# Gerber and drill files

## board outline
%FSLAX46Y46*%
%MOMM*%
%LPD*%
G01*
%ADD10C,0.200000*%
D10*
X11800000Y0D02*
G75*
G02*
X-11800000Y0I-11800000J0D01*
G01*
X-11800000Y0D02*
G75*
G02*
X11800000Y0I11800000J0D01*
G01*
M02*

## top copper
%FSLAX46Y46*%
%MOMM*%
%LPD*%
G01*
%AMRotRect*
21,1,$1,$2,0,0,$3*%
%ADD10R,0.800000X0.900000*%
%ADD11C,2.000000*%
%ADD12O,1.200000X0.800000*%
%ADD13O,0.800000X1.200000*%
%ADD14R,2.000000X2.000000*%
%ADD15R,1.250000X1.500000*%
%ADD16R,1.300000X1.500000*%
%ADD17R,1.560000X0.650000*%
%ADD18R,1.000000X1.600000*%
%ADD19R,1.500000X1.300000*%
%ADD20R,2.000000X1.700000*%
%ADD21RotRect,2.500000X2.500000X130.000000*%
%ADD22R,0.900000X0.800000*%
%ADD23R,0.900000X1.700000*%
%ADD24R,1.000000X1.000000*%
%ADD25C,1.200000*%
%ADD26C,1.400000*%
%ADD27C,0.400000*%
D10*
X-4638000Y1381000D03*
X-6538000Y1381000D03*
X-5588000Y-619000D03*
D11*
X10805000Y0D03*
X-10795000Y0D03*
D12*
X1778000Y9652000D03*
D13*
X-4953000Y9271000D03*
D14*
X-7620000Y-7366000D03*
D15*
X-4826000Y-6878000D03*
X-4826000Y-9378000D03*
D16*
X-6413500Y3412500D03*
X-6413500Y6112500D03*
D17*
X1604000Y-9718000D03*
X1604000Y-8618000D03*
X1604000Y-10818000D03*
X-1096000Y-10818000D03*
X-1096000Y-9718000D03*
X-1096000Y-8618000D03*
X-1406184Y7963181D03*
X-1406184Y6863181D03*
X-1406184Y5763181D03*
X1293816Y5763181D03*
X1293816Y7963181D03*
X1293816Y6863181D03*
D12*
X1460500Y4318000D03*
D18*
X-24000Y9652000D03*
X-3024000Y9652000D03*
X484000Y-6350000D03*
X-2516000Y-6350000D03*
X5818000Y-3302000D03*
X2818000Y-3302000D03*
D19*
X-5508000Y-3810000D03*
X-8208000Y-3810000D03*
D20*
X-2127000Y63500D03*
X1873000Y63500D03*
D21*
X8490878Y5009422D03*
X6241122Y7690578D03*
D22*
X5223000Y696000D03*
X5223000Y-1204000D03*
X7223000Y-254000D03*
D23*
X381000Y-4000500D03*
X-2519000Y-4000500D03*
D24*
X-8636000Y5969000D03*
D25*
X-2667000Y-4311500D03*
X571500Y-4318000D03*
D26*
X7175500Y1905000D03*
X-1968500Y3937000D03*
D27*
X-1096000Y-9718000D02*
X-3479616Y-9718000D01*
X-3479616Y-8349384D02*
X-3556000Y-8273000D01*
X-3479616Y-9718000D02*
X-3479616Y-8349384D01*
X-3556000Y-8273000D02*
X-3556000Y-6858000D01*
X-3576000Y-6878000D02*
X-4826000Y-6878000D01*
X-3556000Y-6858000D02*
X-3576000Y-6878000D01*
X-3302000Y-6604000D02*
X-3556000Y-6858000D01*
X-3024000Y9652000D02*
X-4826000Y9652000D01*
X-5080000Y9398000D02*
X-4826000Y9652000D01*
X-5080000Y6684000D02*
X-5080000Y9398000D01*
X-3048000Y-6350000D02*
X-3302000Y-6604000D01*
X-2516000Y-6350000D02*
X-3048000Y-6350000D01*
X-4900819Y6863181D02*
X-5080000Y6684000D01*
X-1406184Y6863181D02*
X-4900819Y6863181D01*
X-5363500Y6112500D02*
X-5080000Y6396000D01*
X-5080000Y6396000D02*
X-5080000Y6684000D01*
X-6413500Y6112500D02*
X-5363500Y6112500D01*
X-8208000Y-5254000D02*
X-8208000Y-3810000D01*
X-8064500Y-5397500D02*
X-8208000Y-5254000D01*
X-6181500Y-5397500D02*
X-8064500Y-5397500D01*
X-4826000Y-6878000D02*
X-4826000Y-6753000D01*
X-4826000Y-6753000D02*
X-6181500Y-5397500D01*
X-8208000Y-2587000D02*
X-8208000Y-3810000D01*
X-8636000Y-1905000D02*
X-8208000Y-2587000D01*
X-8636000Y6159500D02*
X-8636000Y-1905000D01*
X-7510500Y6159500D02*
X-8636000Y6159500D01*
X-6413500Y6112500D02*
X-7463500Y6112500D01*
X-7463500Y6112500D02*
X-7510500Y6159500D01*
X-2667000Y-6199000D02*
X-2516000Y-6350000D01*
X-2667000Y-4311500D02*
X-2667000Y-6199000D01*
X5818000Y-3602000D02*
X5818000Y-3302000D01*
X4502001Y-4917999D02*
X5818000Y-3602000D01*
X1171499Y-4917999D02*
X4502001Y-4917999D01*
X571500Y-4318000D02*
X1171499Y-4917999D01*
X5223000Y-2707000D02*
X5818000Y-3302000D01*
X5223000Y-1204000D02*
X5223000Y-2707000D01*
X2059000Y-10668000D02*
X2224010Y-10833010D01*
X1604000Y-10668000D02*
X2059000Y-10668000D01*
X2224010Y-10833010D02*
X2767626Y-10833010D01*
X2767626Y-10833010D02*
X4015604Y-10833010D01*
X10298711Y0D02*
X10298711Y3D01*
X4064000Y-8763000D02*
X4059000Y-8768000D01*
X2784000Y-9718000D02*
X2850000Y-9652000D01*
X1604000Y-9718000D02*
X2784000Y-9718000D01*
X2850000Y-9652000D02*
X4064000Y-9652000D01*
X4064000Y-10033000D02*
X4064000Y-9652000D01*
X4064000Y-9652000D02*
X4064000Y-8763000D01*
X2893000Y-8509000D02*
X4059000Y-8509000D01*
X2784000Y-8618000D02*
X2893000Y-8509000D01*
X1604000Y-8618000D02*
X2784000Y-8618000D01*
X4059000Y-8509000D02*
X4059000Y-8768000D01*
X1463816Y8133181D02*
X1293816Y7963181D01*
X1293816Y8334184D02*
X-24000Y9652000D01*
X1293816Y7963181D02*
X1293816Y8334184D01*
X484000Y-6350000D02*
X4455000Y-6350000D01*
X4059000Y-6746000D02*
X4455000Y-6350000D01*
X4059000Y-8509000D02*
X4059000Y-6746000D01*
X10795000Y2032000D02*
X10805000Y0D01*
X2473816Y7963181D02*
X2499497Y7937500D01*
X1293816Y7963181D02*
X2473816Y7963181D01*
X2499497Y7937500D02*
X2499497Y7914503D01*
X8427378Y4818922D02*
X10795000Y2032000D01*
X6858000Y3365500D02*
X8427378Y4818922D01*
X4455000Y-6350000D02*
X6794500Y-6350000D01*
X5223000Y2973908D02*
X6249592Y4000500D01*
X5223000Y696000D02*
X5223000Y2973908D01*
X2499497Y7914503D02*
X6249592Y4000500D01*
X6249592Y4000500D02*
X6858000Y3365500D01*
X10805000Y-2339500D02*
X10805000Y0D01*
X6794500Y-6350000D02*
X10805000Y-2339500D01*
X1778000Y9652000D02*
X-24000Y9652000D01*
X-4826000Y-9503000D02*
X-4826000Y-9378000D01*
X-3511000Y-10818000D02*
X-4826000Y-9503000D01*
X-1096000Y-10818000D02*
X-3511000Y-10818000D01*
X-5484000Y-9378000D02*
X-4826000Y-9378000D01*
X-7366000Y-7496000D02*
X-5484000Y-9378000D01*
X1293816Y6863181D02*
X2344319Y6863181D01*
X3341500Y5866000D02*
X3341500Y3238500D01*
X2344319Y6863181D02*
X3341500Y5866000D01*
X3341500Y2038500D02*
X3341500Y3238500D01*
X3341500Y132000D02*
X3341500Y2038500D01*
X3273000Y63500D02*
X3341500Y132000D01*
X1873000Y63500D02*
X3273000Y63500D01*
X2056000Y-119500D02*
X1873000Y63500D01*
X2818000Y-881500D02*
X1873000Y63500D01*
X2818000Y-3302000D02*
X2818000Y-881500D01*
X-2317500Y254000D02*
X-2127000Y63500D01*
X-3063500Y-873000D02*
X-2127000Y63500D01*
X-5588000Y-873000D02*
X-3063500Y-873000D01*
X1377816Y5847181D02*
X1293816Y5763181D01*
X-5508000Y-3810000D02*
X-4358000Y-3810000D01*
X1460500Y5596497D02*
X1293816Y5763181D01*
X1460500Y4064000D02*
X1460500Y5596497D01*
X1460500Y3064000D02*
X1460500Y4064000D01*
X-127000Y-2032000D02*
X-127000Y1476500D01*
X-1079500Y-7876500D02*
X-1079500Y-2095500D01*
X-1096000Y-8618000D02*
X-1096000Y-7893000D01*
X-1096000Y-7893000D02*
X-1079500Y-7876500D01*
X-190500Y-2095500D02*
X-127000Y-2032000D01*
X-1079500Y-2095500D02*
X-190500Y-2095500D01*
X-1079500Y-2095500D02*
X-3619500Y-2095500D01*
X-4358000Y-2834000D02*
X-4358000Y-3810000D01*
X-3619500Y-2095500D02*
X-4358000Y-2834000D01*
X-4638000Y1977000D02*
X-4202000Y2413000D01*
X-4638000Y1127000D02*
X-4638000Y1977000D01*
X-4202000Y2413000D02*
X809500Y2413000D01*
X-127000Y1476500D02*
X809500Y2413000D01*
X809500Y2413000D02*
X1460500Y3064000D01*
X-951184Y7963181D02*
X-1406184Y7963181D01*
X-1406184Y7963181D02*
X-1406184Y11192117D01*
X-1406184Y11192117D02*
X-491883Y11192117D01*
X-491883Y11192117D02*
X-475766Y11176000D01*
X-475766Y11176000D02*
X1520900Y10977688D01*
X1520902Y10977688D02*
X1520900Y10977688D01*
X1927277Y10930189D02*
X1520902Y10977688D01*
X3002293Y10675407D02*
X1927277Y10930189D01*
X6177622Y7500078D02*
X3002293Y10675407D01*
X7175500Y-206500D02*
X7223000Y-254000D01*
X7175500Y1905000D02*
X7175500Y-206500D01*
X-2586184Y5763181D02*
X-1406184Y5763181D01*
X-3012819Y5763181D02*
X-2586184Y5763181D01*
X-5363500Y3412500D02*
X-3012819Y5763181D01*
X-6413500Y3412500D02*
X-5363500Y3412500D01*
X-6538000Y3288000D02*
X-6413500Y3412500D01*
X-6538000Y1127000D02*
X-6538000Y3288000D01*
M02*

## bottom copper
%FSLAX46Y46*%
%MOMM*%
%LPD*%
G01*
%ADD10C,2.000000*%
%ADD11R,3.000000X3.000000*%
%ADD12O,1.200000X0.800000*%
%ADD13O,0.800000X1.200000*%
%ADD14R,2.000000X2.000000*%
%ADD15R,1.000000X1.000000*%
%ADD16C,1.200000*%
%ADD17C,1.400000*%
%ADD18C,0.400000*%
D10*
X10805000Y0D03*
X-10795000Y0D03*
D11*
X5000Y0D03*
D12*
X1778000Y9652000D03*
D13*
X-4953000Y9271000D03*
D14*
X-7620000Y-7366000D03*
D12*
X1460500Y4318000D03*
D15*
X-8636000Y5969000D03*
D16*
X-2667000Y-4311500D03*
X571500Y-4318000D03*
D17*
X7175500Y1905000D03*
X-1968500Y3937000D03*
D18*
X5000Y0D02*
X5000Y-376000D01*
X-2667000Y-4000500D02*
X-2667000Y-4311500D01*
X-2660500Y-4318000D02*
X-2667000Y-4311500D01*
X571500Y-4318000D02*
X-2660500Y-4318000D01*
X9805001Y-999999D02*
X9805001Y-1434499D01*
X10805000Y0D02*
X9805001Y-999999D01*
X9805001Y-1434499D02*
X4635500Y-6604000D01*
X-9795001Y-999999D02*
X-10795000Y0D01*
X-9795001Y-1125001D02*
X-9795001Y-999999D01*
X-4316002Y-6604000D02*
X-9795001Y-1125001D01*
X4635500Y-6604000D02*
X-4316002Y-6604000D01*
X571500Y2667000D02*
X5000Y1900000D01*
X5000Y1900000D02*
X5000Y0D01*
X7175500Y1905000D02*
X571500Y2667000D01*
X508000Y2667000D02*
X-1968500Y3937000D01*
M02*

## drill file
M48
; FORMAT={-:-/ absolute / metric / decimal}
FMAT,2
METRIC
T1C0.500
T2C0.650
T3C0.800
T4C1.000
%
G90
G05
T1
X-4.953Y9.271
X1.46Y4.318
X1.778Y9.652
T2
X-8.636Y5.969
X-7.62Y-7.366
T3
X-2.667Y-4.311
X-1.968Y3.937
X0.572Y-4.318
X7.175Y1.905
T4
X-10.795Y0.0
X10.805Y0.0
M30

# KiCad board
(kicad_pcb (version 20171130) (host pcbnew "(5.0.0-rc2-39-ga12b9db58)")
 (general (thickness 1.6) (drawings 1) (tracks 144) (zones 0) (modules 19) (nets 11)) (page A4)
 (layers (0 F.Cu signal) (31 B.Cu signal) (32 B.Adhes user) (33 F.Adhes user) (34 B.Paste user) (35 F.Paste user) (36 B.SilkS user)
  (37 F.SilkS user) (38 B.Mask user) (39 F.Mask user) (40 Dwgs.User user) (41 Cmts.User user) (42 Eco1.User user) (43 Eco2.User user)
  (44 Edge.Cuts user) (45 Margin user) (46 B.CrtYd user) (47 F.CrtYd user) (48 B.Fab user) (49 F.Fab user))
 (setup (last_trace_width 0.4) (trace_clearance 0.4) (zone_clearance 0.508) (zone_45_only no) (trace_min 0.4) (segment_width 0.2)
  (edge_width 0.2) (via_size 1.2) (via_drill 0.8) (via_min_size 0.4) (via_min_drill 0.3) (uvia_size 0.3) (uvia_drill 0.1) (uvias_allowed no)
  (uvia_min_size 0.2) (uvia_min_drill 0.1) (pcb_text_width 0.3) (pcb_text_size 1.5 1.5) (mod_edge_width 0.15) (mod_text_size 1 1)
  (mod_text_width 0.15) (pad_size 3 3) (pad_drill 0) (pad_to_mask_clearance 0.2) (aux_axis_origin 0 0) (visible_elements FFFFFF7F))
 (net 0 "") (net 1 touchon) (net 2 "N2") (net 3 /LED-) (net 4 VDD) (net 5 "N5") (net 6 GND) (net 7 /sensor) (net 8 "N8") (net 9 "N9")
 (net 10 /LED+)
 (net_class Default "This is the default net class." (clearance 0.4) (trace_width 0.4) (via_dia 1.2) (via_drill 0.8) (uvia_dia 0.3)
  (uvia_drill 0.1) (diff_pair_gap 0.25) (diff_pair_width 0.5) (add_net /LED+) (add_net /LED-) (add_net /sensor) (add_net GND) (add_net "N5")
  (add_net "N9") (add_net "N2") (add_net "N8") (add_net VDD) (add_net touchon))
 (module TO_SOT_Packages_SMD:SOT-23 (layer F.Cu) (at -5.588 -0.381 270)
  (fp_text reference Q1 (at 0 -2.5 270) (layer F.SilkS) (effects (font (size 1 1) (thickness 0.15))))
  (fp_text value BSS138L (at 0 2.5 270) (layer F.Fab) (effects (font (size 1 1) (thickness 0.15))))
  (pad 1 smd rect (at -1 -0.95 270) (size 0.9 0.8) (layers F.Cu F.Paste F.Mask) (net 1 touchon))
  (pad 2 smd rect (at -1 0.95 270) (size 0.9 0.8) (layers F.Cu F.Paste F.Mask) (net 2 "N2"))
  (pad 3 smd rect (at 1 0 270) (size 0.9 0.8) (layers F.Cu F.Paste F.Mask) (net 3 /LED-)))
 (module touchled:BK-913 (layer B.Cu) (at 0.005 0)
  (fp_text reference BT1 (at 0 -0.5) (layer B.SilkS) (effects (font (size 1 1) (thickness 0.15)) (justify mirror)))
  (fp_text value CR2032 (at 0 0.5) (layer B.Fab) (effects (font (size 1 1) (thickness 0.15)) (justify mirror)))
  (pad 1 thru_hole circle (at 10.8 0) (size 2 2) (drill 1) (layers *.Cu *.Mask) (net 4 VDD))
  (pad 1 thru_hole circle (at -10.8 0) (size 2 2) (drill 1) (layers *.Cu *.Mask) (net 4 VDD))
  (pad 2 smd rect (at 0 0) (size 3 3) (layers B.Cu B.Paste B.Mask) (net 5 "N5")))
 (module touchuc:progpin (layer F.Cu) (at 1.778 -9.652 270)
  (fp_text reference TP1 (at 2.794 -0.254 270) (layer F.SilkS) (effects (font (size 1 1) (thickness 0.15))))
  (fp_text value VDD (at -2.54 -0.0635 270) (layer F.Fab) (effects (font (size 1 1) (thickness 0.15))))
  (pad 1 thru_hole oval (at 0 0 270) (size 0.8 1.2) (drill 0.5) (layers *.Cu *.Mask) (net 4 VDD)))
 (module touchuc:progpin (layer F.Cu) (at -4.953 -9.271 180)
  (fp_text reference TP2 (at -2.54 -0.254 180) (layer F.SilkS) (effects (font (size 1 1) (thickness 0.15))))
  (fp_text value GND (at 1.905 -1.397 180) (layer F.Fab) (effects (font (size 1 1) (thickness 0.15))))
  (pad 1 thru_hole oval (at 0 0 180) (size 0.8 1.2) (drill 0.5) (layers *.Cu *.Mask) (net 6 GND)))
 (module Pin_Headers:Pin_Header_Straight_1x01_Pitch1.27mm (layer F.Cu) (at -7.62 7.366)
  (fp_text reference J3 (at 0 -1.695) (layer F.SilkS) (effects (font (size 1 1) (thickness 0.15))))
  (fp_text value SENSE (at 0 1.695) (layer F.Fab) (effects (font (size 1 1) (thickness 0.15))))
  (pad 1 thru_hole rect (at 0 0) (size 2 2) (drill 0.65) (layers *.Cu *.Mask) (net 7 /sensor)))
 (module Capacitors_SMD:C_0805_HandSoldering (layer F.Cu) (at -4.826 8.128 90)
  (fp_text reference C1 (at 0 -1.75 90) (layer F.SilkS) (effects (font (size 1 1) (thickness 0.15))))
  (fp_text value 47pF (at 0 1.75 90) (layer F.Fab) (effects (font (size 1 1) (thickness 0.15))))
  (pad 2 smd rect (at 1.25 0 90) (size 1.5 1.25) (layers F.Cu F.Paste F.Mask) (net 6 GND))
  (pad 1 smd rect (at -1.25 0 90) (size 1.5 1.25) (layers F.Cu F.Paste F.Mask) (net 7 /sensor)))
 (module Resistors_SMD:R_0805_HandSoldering (layer F.Cu) (at -6.4135 -4.7625 90)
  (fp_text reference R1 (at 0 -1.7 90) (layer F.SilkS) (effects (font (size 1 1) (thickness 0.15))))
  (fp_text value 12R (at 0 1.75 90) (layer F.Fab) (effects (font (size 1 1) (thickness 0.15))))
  (pad 1 smd rect (at -1.35 0 90) (size 1.5 1.3) (layers F.Cu F.Paste F.Mask) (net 2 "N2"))
  (pad 2 smd rect (at 1.35 0 90) (size 1.5 1.3) (layers F.Cu F.Paste F.Mask) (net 6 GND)))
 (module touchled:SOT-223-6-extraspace (layer F.Cu) (at 0.254 9.718)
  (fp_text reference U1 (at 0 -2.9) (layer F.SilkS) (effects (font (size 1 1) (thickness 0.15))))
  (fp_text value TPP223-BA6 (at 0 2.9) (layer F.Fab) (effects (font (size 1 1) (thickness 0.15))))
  (pad 5 smd rect (at 1.35 0) (size 1.56 0.65) (layers F.Cu F.Paste F.Mask) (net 4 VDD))
  (pad 6 smd rect (at 1.35 -1.1) (size 1.56 0.65) (layers F.Cu F.Paste F.Mask) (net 4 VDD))
  (pad 4 smd rect (at 1.35 1.1) (size 1.56 0.65) (layers F.Cu F.Paste F.Mask) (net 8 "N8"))
  (pad 3 smd rect (at -1.35 1.1) (size 1.56 0.65) (layers F.Cu F.Paste F.Mask) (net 7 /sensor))
  (pad 2 smd rect (at -1.35 0) (size 1.56 0.65) (layers F.Cu F.Paste F.Mask) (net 6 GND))
  (pad 1 smd rect (at -1.35 -1.1) (size 1.56 0.65) (layers F.Cu F.Paste F.Mask) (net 1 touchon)))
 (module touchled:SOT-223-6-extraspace (layer F.Cu) (at -0.056184 -6.863181)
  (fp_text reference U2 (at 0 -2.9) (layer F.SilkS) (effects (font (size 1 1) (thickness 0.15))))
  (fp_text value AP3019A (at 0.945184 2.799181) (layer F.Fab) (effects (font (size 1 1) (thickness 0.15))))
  (pad 1 smd rect (at -1.35 -1.1) (size 1.56 0.65) (layers F.Cu F.Paste F.Mask) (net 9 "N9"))
  (pad 2 smd rect (at -1.35 0) (size 1.56 0.65) (layers F.Cu F.Paste F.Mask) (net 6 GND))
  (pad 3 smd rect (at -1.35 1.1) (size 1.56 0.65) (layers F.Cu F.Paste F.Mask) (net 2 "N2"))
  (pad 4 smd rect (at 1.35 1.1) (size 1.56 0.65) (layers F.Cu F.Paste F.Mask) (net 1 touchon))
  (pad 6 smd rect (at 1.35 -1.1) (size 1.56 0.65) (layers F.Cu F.Paste F.Mask) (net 4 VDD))
  (pad 5 smd rect (at 1.35 0) (size 1.56 0.65) (layers F.Cu F.Paste F.Mask) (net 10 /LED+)))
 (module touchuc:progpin (layer F.Cu) (at 1.4605 -4.318 90)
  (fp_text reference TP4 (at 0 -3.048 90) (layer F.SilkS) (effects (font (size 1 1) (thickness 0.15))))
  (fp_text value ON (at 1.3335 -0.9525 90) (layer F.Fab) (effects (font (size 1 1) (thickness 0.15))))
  (pad 1 thru_hole oval (at 0 0 90) (size 0.8 1.2) (drill 0.5) (layers *.Cu *.Mask) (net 1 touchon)))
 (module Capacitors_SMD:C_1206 (layer F.Cu) (at -1.524 -9.652 180)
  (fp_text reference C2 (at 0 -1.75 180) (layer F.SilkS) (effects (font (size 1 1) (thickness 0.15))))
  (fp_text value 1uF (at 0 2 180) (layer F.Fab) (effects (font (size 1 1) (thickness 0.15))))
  (pad 1 smd rect (at -1.5 0 180) (size 1 1.6) (layers F.Cu F.Paste F.Mask) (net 4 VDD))
  (pad 2 smd rect (at 1.5 0 180) (size 1 1.6) (layers F.Cu F.Paste F.Mask) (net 6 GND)))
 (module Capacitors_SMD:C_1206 (layer F.Cu) (at -1.016 6.35 180)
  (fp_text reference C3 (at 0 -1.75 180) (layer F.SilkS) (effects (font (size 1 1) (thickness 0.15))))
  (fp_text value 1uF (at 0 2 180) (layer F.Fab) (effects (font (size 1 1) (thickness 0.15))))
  (pad 1 smd rect (at -1.5 0 180) (size 1 1.6) (layers F.Cu F.Paste F.Mask) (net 4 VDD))
  (pad 2 smd rect (at 1.5 0 180) (size 1 1.6) (layers F.Cu F.Paste F.Mask) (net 6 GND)))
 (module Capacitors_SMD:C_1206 (layer F.Cu) (at 4.318 3.302)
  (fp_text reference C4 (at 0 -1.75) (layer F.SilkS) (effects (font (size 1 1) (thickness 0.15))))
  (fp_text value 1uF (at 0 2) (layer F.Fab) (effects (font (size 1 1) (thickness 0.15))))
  (pad 2 smd rect (at 1.5 0) (size 1 1.6) (layers F.Cu F.Paste F.Mask) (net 6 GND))
  (pad 1 smd rect (at -1.5 0) (size 1 1.6) (layers F.Cu F.Paste F.Mask) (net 10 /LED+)))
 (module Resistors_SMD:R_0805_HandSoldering (layer F.Cu) (at -6.858 3.81 180)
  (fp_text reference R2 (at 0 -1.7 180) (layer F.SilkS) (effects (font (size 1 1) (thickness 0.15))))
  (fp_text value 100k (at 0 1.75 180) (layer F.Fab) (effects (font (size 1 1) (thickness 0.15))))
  (pad 1 smd rect (at -1.35 0 180) (size 1.5 1.3) (layers F.Cu F.Paste F.Mask) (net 1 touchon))
  (pad 2 smd rect (at 1.35 0 180) (size 1.5 1.3) (layers F.Cu F.Paste F.Mask) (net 6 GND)))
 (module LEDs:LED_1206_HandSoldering (layer F.Cu) (at -0.127 -0.0635)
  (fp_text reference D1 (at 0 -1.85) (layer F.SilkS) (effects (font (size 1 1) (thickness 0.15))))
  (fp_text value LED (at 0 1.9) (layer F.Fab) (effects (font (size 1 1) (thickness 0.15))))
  (pad 1 smd rect (at -2 0) (size 2 1.7) (layers F.Cu F.Paste F.Mask) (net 3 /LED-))
  (pad 2 smd rect (at 2 0) (size 2 1.7) (layers F.Cu F.Paste F.Mask) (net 10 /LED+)))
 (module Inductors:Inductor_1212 (layer F.Cu) (at 7.366 -6.35 130)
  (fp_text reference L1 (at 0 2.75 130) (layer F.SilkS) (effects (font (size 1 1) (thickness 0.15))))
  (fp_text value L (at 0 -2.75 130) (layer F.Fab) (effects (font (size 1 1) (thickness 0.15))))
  (pad 1 smd rect (at -1.75 0 130) (size 2.5 2.5) (layers F.Cu F.Paste F.Mask) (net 4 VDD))
  (pad 2 smd rect (at 1.75 0 130) (size 2.5 2.5) (layers F.Cu F.Paste F.Mask) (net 9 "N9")))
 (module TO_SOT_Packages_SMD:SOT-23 (layer F.Cu) (at 6.223 0.254)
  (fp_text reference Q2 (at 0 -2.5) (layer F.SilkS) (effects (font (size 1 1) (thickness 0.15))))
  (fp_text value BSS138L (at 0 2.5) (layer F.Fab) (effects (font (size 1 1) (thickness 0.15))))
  (pad 1 smd rect (at -1 -0.95) (size 0.9 0.8) (layers F.Cu F.Paste F.Mask) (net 4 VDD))
  (pad 2 smd rect (at -1 0.95) (size 0.9 0.8) (layers F.Cu F.Paste F.Mask) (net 6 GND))
  (pad 3 smd rect (at 1 0) (size 0.9 0.8) (layers F.Cu F.Paste F.Mask) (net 5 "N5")))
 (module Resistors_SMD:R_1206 (layer F.Cu) (at -1.069 4.0005)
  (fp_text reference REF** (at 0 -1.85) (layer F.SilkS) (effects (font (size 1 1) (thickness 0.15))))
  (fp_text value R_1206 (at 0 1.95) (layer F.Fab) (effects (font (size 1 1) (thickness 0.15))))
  (pad 2 smd rect (at 1.45 0) (size 0.9 1.7) (layers F.Cu F.Paste F.Mask))
  (pad 1 smd rect (at -1.45 0) (size 0.9 1.7) (layers F.Cu F.Paste F.Mask)))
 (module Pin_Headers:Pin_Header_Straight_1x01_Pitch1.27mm (layer F.Cu) (at -8.636 -5.969)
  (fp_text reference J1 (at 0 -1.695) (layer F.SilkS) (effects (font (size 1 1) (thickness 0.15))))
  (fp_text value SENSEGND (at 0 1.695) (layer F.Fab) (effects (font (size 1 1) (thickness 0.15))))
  (pad 1 thru_hole rect (at 0 0) (size 1 1) (drill 0.65) (layers *.Cu *.Mask) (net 6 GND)))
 (gr_circle (center 0 0) (end 11.8 0) (layer Edge.Cuts) (width 0.2))
 (segment (start -1.096 9.718) (end -3.479616 9.718) (width 0.4) (layer F.Cu) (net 6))
 (segment (start -3.479616 8.349384) (end -3.556 8.273) (width 0.4) (layer F.Cu) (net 6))
 (segment (start -3.479616 9.718) (end -3.479616 8.349384) (width 0.4) (layer F.Cu) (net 6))
 (segment (start -3.556 8.273) (end -3.556 6.858) (width 0.4) (layer F.Cu) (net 6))
 (segment (start -3.576 6.878) (end -4.826 6.878) (width 0.4) (layer F.Cu) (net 6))
 (segment (start -3.556 6.858) (end -3.576 6.878) (width 0.4) (layer F.Cu) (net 6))
 (segment (start -3.302 6.604) (end -3.556 6.858) (width 0.4) (layer F.Cu) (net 6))
 (segment (start -3.024 -9.652) (end -4.826 -9.652) (width 0.4) (layer F.Cu) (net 6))
 (segment (start -5.08 -9.398) (end -4.826 -9.652) (width 0.4) (layer F.Cu) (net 6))
 (segment (start -5.08 -6.684) (end -5.08 -9.398) (width 0.4) (layer F.Cu) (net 6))
 (segment (start -3.048 6.35) (end -3.302 6.604) (width 0.4) (layer F.Cu) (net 6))
 (segment (start -2.516 6.35) (end -3.048 6.35) (width 0.4) (layer F.Cu) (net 6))
 (segment (start -4.900819 -6.863181) (end -5.08 -6.684) (width 0.4) (layer F.Cu) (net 6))
 (segment (start -1.406184 -6.863181) (end -4.900819 -6.863181) (width 0.4) (layer F.Cu) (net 6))
 (segment (start -5.3635 -6.1125) (end -5.08 -6.396) (width 0.4) (layer F.Cu) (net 6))
 (segment (start -5.08 -6.396) (end -5.08 -6.684) (width 0.4) (layer F.Cu) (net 6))
 (segment (start -6.4135 -6.1125) (end -5.3635 -6.1125) (width 0.4) (layer F.Cu) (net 6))
 (segment (start -8.208 5.254) (end -8.208 3.81) (width 0.4) (layer F.Cu) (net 6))
 (segment (start -8.0645 5.3975) (end -8.208 5.254) (width 0.4) (layer F.Cu) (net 6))
 (segment (start -6.1815 5.3975) (end -8.0645 5.3975) (width 0.4) (layer F.Cu) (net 6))
 (segment (start -4.826 6.878) (end -4.826 6.753) (width 0.4) (layer F.Cu) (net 6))
 (segment (start -4.826 6.753) (end -6.1815 5.3975) (width 0.4) (layer F.Cu) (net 6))
 (segment (start -8.208 2.587) (end -8.208 3.81) (width 0.4) (layer F.Cu) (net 6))
 (segment (start -8.636 1.905) (end -8.208 2.587) (width 0.4) (layer F.Cu) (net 6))
 (segment (start -8.636 -6.1595) (end -8.636 1.905) (width 0.4) (layer F.Cu) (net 6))
 (segment (start -7.5105 -6.1595) (end -8.636 -6.1595) (width 0.4) (layer F.Cu) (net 6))
 (segment (start -6.4135 -6.1125) (end -7.4635 -6.1125) (width 0.4) (layer F.Cu) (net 6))
 (segment (start -7.4635 -6.1125) (end -7.5105 -6.1595) (width 0.4) (layer F.Cu) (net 6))
 (segment (start 0.005 0) (end 0.005 0.376) (width 0.4) (layer B.Cu) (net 5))
 (segment (start -2.667 6.199) (end -2.516 6.35) (width 0.4) (layer F.Cu) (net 6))
 (segment (start -2.667 4.3115) (end -2.667 6.199) (width 0.4) (layer F.Cu) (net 6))
 (segment (start -2.667 4.0005) (end -2.667 4.3115) (width 0.4) (layer B.Cu) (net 6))
 (via (at -2.667 4.3115) (size 1.2) (drill 0.8) (layers F.Cu B.Cu) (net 6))
 (via (at 0.5715 4.318) (size 1.2) (drill 0.8) (layers F.Cu B.Cu) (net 6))
 (segment (start -2.6605 4.318) (end -2.667 4.3115) (width 0.4) (layer B.Cu) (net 6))
 (segment (start 0.5715 4.318) (end -2.6605 4.318) (width 0.4) (layer B.Cu) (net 6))
 (segment (start 5.818 3.602) (end 5.818 3.302) (width 0.4) (layer F.Cu) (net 6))
 (segment (start 4.502001 4.917999) (end 5.818 3.602) (width 0.4) (layer F.Cu) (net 6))
 (segment (start 1.171499 4.917999) (end 4.502001 4.917999) (width 0.4) (layer F.Cu) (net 6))
 (segment (start 0.5715 4.318) (end 1.171499 4.917999) (width 0.4) (layer F.Cu) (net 6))
 (segment (start 5.223 2.707) (end 5.818 3.302) (width 0.4) (layer F.Cu) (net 6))
 (segment (start 5.223 1.204) (end 5.223 2.707) (width 0.4) (layer F.Cu) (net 6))
 (segment (start 2.059 10.668) (end 2.22401 10.83301) (width 0.4) (layer F.Cu) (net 8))
 (segment (start 1.604 10.668) (end 2.059 10.668) (width 0.4) (layer F.Cu) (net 8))
 (segment (start 2.22401 10.83301) (end 2.767626 10.83301) (width 0.4) (layer F.Cu) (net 8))
 (segment (start 2.767626 10.83301) (end 4.015604 10.83301) (width 0.4) (layer F.Cu) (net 8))
 (segment (start 10.298711 0) (end 10.298711 -0.000003) (width 0.4) (layer F.Cu) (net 4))
 (segment (start 4.064 8.763) (end 4.059 8.768) (width 0.4) (layer F.Cu) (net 4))
 (segment (start 2.784 9.718) (end 2.85 9.652) (width 0.4) (layer F.Cu) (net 4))
 (segment (start 1.604 9.718) (end 2.784 9.718) (width 0.4) (layer F.Cu) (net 4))
 (segment (start 2.85 9.652) (end 4.064 9.652) (width 0.4) (layer F.Cu) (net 4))
 (segment (start 4.064 10.033) (end 4.064 9.652) (width 0.4) (layer F.Cu) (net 4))
 (segment (start 4.064 9.652) (end 4.064 8.763) (width 0.4) (layer F.Cu) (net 4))
 (segment (start 2.893 8.509) (end 4.059 8.509) (width 0.4) (layer F.Cu) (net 4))
 (segment (start 2.784 8.618) (end 2.893 8.509) (width 0.4) (layer F.Cu) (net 4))
 (segment (start 1.604 8.618) (end 2.784 8.618) (width 0.4) (layer F.Cu) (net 4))
 (segment (start 4.059 8.509) (end 4.059 8.768) (width 0.4) (layer F.Cu) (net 4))
 (segment (start 1.463816 -8.133181) (end 1.293816 -7.963181) (width 0.4) (layer F.Cu) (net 4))
 (segment (start 1.293816 -8.334184) (end -0.024 -9.652) (width 0.4) (layer F.Cu) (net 4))
 (segment (start 1.293816 -7.963181) (end 1.293816 -8.334184) (width 0.4) (layer F.Cu) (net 4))
 (segment (start 0.484 6.35) (end 4.455 6.35) (width 0.4) (layer F.Cu) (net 4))
 (segment (start 4.059 6.746) (end 4.455 6.35) (width 0.4) (layer F.Cu) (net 4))
 (segment (start 4.059 8.509) (end 4.059 6.746) (width 0.4) (layer F.Cu) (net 4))
 (segment (start 9.805001 0.999999) (end 9.805001 1.434499) (width 0.4) (layer B.Cu) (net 4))
 (segment (start 10.805 0) (end 9.805001 0.999999) (width 0.4) (layer B.Cu) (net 4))
 (segment (start 9.805001 1.434499) (end 4.6355 6.604) (width 0.4) (layer B.Cu) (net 4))
 (segment (start -9.795001 0.999999) (end -10.795 0) (width 0.4) (layer B.Cu) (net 4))
 (segment (start -9.795001 1.125001) (end -9.795001 0.999999) (width 0.4) (layer B.Cu) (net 4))
 (segment (start -4.316002 6.604) (end -9.795001 1.125001) (width 0.4) (layer B.Cu) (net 4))
 (segment (start 4.6355 6.604) (end -4.316002 6.604) (width 0.4) (layer B.Cu) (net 4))
 (segment (start 10.795 -2.032) (end 10.805 0) (width 0.4) (layer F.Cu) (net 4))
 (segment (start 2.473816 -7.963181) (end 2.499497 -7.9375) (width 0.4) (layer F.Cu) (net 4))
 (segment (start 1.293816 -7.963181) (end 2.473816 -7.963181) (width 0.4) (layer F.Cu) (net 4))
 (segment (start 2.499497 -7.9375) (end 2.499497 -7.914503) (width 0.4) (layer F.Cu) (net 4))
 (segment (start 8.427378 -4.818922) (end 10.795 -2.032) (width 0.4) (layer F.Cu) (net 4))
 (segment (start 6.858 -3.3655) (end 8.427378 -4.818922) (width 0.4) (layer F.Cu) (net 4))
 (segment (start 4.455 6.35) (end 6.7945 6.35) (width 0.4) (layer F.Cu) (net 4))
 (segment (start 5.223 -2.973908) (end 6.249592 -4.0005) (width 0.4) (layer F.Cu) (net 4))
 (segment (start 5.223 -0.696) (end 5.223 -2.973908) (width 0.4) (layer F.Cu) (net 4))
 (segment (start 2.499497 -7.914503) (end 6.249592 -4.0005) (width 0.4) (layer F.Cu) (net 4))
 (segment (start 6.249592 -4.0005) (end 6.858 -3.3655) (width 0.4) (layer F.Cu) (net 4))
 (segment (start 10.805 2.3395) (end 10.805 0) (width 0.4) (layer F.Cu) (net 4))
 (segment (start 6.7945 6.35) (end 10.805 2.3395) (width 0.4) (layer F.Cu) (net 4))
 (segment (start 1.778 -9.652) (end -0.024 -9.652) (width 0.4) (layer F.Cu) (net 4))
 (segment (start -4.826 9.503) (end -4.826 9.378) (width 0.4) (layer F.Cu) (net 7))
 (segment (start -3.511 10.818) (end -4.826 9.503) (width 0.4) (layer F.Cu) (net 7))
 (segment (start -1.096 10.818) (end -3.511 10.818) (width 0.4) (layer F.Cu) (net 7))
 (segment (start -5.484 9.378) (end -4.826 9.378) (width 0.4) (layer F.Cu) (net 7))
 (segment (start -7.366 7.496) (end -5.484 9.378) (width 0.4) (layer F.Cu) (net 7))
 (segment (start 1.293816 -6.863181) (end 2.344319 -6.863181) (width 0.4) (layer F.Cu) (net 10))
 (segment (start 3.3415 -5.866) (end 3.3415 -3.2385) (width 0.4) (layer F.Cu) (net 10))
 (segment (start 2.344319 -6.863181) (end 3.3415 -5.866) (width 0.4) (layer F.Cu) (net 10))
 (segment (start 3.3415 -2.0385) (end 3.3415 -3.2385) (width 0.4) (layer F.Cu) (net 10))
 (segment (start 3.3415 -0.132) (end 3.3415 -2.0385) (width 0.4) (layer F.Cu) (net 10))
 (segment (start 3.273 -0.0635) (end 3.3415 -0.132) (width 0.4) (layer F.Cu) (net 10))
 (segment (start 1.873 -0.0635) (end 3.273 -0.0635) (width 0.4) (layer F.Cu) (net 10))
 (segment (start 2.056 0.1195) (end 1.873 -0.0635) (width 0.4) (layer F.Cu) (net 10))
 (segment (start 2.818 0.8815) (end 1.873 -0.0635) (width 0.4) (layer F.Cu) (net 10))
 (segment (start 2.818 3.302) (end 2.818 0.8815) (width 0.4) (layer F.Cu) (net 10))
 (segment (start -2.3175 -0.254) (end -2.127 -0.0635) (width 0.4) (layer F.Cu) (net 3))
 (segment (start -3.0635 0.873) (end -2.127 -0.0635) (width 0.4) (layer F.Cu) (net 3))
 (segment (start -5.588 0.873) (end -3.0635 0.873) (width 0.4) (layer F.Cu) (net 3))
 (segment (start 1.377816 -5.847181) (end 1.293816 -5.763181) (width 0.4) (layer F.Cu) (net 1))
 (segment (start -5.508 3.81) (end -4.358 3.81) (width 0.4) (layer F.Cu) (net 1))
 (segment (start 1.4605 -5.596497) (end 1.293816 -5.763181) (width 0.4) (layer F.Cu) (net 1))
 (segment (start 1.4605 -4.064) (end 1.4605 -5.596497) (width 0.4) (layer F.Cu) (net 1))
 (segment (start 1.4605 -3.064) (end 1.4605 -4.064) (width 0.4) (layer F.Cu) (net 1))
 (segment (start -0.127 2.032) (end -0.127 -1.4765) (width 0.4) (layer F.Cu) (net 1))
 (segment (start -1.0795 7.8765) (end -1.0795 2.0955) (width 0.4) (layer F.Cu) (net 1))
 (segment (start -1.096 8.618) (end -1.096 7.893) (width 0.4) (layer F.Cu) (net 1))
 (segment (start -1.096 7.893) (end -1.0795 7.8765) (width 0.4) (layer F.Cu) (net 1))
 (segment (start -0.1905 2.0955) (end -0.127 2.032) (width 0.4) (layer F.Cu) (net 1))
 (segment (start -1.0795 2.0955) (end -0.1905 2.0955) (width 0.4) (layer F.Cu) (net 1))
 (segment (start -1.0795 2.0955) (end -3.6195 2.0955) (width 0.4) (layer F.Cu) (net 1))
 (segment (start -4.358 2.834) (end -4.358 3.81) (width 0.4) (layer F.Cu) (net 1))
 (segment (start -3.6195 2.0955) (end -4.358 2.834) (width 0.4) (layer F.Cu) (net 1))
 (segment (start -4.638 -1.977) (end -4.202 -2.413) (width 0.4) (layer F.Cu) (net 1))
 (segment (start -4.638 -1.127) (end -4.638 -1.977) (width 0.4) (layer F.Cu) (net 1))
 (segment (start -4.202 -2.413) (end 0.8095 -2.413) (width 0.4) (layer F.Cu) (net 1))
 (segment (start -0.127 -1.4765) (end 0.8095 -2.413) (width 0.4) (layer F.Cu) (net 1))
 (segment (start 0.8095 -2.413) (end 1.4605 -3.064) (width 0.4) (layer F.Cu) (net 1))
 (segment (start -0.951184 -7.963181) (end -1.406184 -7.963181) (width 0.4) (layer F.Cu) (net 9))
 (segment (start -1.406184 -7.963181) (end -1.406184 -11.192117) (width 0.4) (layer F.Cu) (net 9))
 (segment (start -1.406184 -11.192117) (end -0.491883 -11.192117) (width 0.4) (layer F.Cu) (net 9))
 (segment (start -0.491883 -11.192117) (end -0.475766 -11.176) (width 0.4) (layer F.Cu) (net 9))
 (segment (start -0.475766 -11.176) (end 1.5209 -10.977688) (width 0.4) (layer F.Cu) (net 9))
 (segment (start 1.520902 -10.977688) (end 1.5209 -10.977688) (width 0.4) (layer F.Cu) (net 9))
 (segment (start 1.927277 -10.930189) (end 1.520902 -10.977688) (width 0.4) (layer F.Cu) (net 9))
 (segment (start 3.002293 -10.675407) (end 1.927277 -10.930189) (width 0.4) (layer F.Cu) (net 9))
 (segment (start 6.177622 -7.500078) (end 3.002293 -10.675407) (width 0.4) (layer F.Cu) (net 9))
 (segment (start 0.5715 -2.667) (end 0.005 -1.9) (width 0.4) (layer B.Cu) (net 5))
 (segment (start 0.005 -1.9) (end 0.005 0) (width 0.4) (layer B.Cu) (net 5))
 (via (at 7.1755 -1.905) (size 1.4) (drill 0.8) (layers F.Cu B.Cu) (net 5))
 (segment (start 7.1755 -1.905) (end 0.5715 -2.667) (width 0.4) (layer B.Cu) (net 5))
 (segment (start 7.1755 0.2065) (end 7.223 0.254) (width 0.4) (layer F.Cu) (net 5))
 (segment (start 7.1755 -1.905) (end 7.1755 0.2065) (width 0.4) (layer F.Cu) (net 5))
 (segment (start 0.508 -2.667) (end -1.9685 -3.937) (width 0.4) (layer B.Cu) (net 5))
 (via (at -1.9685 -3.937) (size 1.4) (drill 0.8) (layers F.Cu B.Cu) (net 5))
 (segment (start -2.586184 -5.763181) (end -1.406184 -5.763181) (width 0.4) (layer F.Cu) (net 2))
 (segment (start -3.012819 -5.763181) (end -2.586184 -5.763181) (width 0.4) (layer F.Cu) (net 2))
 (segment (start -5.3635 -3.4125) (end -3.012819 -5.763181) (width 0.4) (layer F.Cu) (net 2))
 (segment (start -6.4135 -3.4125) (end -5.3635 -3.4125) (width 0.4) (layer F.Cu) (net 2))
 (segment (start -6.538 -3.288) (end -6.4135 -3.4125) (width 0.4) (layer F.Cu) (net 2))
 (segment (start -6.538 -1.127) (end -6.538 -3.288) (width 0.4) (layer F.Cu) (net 2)))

